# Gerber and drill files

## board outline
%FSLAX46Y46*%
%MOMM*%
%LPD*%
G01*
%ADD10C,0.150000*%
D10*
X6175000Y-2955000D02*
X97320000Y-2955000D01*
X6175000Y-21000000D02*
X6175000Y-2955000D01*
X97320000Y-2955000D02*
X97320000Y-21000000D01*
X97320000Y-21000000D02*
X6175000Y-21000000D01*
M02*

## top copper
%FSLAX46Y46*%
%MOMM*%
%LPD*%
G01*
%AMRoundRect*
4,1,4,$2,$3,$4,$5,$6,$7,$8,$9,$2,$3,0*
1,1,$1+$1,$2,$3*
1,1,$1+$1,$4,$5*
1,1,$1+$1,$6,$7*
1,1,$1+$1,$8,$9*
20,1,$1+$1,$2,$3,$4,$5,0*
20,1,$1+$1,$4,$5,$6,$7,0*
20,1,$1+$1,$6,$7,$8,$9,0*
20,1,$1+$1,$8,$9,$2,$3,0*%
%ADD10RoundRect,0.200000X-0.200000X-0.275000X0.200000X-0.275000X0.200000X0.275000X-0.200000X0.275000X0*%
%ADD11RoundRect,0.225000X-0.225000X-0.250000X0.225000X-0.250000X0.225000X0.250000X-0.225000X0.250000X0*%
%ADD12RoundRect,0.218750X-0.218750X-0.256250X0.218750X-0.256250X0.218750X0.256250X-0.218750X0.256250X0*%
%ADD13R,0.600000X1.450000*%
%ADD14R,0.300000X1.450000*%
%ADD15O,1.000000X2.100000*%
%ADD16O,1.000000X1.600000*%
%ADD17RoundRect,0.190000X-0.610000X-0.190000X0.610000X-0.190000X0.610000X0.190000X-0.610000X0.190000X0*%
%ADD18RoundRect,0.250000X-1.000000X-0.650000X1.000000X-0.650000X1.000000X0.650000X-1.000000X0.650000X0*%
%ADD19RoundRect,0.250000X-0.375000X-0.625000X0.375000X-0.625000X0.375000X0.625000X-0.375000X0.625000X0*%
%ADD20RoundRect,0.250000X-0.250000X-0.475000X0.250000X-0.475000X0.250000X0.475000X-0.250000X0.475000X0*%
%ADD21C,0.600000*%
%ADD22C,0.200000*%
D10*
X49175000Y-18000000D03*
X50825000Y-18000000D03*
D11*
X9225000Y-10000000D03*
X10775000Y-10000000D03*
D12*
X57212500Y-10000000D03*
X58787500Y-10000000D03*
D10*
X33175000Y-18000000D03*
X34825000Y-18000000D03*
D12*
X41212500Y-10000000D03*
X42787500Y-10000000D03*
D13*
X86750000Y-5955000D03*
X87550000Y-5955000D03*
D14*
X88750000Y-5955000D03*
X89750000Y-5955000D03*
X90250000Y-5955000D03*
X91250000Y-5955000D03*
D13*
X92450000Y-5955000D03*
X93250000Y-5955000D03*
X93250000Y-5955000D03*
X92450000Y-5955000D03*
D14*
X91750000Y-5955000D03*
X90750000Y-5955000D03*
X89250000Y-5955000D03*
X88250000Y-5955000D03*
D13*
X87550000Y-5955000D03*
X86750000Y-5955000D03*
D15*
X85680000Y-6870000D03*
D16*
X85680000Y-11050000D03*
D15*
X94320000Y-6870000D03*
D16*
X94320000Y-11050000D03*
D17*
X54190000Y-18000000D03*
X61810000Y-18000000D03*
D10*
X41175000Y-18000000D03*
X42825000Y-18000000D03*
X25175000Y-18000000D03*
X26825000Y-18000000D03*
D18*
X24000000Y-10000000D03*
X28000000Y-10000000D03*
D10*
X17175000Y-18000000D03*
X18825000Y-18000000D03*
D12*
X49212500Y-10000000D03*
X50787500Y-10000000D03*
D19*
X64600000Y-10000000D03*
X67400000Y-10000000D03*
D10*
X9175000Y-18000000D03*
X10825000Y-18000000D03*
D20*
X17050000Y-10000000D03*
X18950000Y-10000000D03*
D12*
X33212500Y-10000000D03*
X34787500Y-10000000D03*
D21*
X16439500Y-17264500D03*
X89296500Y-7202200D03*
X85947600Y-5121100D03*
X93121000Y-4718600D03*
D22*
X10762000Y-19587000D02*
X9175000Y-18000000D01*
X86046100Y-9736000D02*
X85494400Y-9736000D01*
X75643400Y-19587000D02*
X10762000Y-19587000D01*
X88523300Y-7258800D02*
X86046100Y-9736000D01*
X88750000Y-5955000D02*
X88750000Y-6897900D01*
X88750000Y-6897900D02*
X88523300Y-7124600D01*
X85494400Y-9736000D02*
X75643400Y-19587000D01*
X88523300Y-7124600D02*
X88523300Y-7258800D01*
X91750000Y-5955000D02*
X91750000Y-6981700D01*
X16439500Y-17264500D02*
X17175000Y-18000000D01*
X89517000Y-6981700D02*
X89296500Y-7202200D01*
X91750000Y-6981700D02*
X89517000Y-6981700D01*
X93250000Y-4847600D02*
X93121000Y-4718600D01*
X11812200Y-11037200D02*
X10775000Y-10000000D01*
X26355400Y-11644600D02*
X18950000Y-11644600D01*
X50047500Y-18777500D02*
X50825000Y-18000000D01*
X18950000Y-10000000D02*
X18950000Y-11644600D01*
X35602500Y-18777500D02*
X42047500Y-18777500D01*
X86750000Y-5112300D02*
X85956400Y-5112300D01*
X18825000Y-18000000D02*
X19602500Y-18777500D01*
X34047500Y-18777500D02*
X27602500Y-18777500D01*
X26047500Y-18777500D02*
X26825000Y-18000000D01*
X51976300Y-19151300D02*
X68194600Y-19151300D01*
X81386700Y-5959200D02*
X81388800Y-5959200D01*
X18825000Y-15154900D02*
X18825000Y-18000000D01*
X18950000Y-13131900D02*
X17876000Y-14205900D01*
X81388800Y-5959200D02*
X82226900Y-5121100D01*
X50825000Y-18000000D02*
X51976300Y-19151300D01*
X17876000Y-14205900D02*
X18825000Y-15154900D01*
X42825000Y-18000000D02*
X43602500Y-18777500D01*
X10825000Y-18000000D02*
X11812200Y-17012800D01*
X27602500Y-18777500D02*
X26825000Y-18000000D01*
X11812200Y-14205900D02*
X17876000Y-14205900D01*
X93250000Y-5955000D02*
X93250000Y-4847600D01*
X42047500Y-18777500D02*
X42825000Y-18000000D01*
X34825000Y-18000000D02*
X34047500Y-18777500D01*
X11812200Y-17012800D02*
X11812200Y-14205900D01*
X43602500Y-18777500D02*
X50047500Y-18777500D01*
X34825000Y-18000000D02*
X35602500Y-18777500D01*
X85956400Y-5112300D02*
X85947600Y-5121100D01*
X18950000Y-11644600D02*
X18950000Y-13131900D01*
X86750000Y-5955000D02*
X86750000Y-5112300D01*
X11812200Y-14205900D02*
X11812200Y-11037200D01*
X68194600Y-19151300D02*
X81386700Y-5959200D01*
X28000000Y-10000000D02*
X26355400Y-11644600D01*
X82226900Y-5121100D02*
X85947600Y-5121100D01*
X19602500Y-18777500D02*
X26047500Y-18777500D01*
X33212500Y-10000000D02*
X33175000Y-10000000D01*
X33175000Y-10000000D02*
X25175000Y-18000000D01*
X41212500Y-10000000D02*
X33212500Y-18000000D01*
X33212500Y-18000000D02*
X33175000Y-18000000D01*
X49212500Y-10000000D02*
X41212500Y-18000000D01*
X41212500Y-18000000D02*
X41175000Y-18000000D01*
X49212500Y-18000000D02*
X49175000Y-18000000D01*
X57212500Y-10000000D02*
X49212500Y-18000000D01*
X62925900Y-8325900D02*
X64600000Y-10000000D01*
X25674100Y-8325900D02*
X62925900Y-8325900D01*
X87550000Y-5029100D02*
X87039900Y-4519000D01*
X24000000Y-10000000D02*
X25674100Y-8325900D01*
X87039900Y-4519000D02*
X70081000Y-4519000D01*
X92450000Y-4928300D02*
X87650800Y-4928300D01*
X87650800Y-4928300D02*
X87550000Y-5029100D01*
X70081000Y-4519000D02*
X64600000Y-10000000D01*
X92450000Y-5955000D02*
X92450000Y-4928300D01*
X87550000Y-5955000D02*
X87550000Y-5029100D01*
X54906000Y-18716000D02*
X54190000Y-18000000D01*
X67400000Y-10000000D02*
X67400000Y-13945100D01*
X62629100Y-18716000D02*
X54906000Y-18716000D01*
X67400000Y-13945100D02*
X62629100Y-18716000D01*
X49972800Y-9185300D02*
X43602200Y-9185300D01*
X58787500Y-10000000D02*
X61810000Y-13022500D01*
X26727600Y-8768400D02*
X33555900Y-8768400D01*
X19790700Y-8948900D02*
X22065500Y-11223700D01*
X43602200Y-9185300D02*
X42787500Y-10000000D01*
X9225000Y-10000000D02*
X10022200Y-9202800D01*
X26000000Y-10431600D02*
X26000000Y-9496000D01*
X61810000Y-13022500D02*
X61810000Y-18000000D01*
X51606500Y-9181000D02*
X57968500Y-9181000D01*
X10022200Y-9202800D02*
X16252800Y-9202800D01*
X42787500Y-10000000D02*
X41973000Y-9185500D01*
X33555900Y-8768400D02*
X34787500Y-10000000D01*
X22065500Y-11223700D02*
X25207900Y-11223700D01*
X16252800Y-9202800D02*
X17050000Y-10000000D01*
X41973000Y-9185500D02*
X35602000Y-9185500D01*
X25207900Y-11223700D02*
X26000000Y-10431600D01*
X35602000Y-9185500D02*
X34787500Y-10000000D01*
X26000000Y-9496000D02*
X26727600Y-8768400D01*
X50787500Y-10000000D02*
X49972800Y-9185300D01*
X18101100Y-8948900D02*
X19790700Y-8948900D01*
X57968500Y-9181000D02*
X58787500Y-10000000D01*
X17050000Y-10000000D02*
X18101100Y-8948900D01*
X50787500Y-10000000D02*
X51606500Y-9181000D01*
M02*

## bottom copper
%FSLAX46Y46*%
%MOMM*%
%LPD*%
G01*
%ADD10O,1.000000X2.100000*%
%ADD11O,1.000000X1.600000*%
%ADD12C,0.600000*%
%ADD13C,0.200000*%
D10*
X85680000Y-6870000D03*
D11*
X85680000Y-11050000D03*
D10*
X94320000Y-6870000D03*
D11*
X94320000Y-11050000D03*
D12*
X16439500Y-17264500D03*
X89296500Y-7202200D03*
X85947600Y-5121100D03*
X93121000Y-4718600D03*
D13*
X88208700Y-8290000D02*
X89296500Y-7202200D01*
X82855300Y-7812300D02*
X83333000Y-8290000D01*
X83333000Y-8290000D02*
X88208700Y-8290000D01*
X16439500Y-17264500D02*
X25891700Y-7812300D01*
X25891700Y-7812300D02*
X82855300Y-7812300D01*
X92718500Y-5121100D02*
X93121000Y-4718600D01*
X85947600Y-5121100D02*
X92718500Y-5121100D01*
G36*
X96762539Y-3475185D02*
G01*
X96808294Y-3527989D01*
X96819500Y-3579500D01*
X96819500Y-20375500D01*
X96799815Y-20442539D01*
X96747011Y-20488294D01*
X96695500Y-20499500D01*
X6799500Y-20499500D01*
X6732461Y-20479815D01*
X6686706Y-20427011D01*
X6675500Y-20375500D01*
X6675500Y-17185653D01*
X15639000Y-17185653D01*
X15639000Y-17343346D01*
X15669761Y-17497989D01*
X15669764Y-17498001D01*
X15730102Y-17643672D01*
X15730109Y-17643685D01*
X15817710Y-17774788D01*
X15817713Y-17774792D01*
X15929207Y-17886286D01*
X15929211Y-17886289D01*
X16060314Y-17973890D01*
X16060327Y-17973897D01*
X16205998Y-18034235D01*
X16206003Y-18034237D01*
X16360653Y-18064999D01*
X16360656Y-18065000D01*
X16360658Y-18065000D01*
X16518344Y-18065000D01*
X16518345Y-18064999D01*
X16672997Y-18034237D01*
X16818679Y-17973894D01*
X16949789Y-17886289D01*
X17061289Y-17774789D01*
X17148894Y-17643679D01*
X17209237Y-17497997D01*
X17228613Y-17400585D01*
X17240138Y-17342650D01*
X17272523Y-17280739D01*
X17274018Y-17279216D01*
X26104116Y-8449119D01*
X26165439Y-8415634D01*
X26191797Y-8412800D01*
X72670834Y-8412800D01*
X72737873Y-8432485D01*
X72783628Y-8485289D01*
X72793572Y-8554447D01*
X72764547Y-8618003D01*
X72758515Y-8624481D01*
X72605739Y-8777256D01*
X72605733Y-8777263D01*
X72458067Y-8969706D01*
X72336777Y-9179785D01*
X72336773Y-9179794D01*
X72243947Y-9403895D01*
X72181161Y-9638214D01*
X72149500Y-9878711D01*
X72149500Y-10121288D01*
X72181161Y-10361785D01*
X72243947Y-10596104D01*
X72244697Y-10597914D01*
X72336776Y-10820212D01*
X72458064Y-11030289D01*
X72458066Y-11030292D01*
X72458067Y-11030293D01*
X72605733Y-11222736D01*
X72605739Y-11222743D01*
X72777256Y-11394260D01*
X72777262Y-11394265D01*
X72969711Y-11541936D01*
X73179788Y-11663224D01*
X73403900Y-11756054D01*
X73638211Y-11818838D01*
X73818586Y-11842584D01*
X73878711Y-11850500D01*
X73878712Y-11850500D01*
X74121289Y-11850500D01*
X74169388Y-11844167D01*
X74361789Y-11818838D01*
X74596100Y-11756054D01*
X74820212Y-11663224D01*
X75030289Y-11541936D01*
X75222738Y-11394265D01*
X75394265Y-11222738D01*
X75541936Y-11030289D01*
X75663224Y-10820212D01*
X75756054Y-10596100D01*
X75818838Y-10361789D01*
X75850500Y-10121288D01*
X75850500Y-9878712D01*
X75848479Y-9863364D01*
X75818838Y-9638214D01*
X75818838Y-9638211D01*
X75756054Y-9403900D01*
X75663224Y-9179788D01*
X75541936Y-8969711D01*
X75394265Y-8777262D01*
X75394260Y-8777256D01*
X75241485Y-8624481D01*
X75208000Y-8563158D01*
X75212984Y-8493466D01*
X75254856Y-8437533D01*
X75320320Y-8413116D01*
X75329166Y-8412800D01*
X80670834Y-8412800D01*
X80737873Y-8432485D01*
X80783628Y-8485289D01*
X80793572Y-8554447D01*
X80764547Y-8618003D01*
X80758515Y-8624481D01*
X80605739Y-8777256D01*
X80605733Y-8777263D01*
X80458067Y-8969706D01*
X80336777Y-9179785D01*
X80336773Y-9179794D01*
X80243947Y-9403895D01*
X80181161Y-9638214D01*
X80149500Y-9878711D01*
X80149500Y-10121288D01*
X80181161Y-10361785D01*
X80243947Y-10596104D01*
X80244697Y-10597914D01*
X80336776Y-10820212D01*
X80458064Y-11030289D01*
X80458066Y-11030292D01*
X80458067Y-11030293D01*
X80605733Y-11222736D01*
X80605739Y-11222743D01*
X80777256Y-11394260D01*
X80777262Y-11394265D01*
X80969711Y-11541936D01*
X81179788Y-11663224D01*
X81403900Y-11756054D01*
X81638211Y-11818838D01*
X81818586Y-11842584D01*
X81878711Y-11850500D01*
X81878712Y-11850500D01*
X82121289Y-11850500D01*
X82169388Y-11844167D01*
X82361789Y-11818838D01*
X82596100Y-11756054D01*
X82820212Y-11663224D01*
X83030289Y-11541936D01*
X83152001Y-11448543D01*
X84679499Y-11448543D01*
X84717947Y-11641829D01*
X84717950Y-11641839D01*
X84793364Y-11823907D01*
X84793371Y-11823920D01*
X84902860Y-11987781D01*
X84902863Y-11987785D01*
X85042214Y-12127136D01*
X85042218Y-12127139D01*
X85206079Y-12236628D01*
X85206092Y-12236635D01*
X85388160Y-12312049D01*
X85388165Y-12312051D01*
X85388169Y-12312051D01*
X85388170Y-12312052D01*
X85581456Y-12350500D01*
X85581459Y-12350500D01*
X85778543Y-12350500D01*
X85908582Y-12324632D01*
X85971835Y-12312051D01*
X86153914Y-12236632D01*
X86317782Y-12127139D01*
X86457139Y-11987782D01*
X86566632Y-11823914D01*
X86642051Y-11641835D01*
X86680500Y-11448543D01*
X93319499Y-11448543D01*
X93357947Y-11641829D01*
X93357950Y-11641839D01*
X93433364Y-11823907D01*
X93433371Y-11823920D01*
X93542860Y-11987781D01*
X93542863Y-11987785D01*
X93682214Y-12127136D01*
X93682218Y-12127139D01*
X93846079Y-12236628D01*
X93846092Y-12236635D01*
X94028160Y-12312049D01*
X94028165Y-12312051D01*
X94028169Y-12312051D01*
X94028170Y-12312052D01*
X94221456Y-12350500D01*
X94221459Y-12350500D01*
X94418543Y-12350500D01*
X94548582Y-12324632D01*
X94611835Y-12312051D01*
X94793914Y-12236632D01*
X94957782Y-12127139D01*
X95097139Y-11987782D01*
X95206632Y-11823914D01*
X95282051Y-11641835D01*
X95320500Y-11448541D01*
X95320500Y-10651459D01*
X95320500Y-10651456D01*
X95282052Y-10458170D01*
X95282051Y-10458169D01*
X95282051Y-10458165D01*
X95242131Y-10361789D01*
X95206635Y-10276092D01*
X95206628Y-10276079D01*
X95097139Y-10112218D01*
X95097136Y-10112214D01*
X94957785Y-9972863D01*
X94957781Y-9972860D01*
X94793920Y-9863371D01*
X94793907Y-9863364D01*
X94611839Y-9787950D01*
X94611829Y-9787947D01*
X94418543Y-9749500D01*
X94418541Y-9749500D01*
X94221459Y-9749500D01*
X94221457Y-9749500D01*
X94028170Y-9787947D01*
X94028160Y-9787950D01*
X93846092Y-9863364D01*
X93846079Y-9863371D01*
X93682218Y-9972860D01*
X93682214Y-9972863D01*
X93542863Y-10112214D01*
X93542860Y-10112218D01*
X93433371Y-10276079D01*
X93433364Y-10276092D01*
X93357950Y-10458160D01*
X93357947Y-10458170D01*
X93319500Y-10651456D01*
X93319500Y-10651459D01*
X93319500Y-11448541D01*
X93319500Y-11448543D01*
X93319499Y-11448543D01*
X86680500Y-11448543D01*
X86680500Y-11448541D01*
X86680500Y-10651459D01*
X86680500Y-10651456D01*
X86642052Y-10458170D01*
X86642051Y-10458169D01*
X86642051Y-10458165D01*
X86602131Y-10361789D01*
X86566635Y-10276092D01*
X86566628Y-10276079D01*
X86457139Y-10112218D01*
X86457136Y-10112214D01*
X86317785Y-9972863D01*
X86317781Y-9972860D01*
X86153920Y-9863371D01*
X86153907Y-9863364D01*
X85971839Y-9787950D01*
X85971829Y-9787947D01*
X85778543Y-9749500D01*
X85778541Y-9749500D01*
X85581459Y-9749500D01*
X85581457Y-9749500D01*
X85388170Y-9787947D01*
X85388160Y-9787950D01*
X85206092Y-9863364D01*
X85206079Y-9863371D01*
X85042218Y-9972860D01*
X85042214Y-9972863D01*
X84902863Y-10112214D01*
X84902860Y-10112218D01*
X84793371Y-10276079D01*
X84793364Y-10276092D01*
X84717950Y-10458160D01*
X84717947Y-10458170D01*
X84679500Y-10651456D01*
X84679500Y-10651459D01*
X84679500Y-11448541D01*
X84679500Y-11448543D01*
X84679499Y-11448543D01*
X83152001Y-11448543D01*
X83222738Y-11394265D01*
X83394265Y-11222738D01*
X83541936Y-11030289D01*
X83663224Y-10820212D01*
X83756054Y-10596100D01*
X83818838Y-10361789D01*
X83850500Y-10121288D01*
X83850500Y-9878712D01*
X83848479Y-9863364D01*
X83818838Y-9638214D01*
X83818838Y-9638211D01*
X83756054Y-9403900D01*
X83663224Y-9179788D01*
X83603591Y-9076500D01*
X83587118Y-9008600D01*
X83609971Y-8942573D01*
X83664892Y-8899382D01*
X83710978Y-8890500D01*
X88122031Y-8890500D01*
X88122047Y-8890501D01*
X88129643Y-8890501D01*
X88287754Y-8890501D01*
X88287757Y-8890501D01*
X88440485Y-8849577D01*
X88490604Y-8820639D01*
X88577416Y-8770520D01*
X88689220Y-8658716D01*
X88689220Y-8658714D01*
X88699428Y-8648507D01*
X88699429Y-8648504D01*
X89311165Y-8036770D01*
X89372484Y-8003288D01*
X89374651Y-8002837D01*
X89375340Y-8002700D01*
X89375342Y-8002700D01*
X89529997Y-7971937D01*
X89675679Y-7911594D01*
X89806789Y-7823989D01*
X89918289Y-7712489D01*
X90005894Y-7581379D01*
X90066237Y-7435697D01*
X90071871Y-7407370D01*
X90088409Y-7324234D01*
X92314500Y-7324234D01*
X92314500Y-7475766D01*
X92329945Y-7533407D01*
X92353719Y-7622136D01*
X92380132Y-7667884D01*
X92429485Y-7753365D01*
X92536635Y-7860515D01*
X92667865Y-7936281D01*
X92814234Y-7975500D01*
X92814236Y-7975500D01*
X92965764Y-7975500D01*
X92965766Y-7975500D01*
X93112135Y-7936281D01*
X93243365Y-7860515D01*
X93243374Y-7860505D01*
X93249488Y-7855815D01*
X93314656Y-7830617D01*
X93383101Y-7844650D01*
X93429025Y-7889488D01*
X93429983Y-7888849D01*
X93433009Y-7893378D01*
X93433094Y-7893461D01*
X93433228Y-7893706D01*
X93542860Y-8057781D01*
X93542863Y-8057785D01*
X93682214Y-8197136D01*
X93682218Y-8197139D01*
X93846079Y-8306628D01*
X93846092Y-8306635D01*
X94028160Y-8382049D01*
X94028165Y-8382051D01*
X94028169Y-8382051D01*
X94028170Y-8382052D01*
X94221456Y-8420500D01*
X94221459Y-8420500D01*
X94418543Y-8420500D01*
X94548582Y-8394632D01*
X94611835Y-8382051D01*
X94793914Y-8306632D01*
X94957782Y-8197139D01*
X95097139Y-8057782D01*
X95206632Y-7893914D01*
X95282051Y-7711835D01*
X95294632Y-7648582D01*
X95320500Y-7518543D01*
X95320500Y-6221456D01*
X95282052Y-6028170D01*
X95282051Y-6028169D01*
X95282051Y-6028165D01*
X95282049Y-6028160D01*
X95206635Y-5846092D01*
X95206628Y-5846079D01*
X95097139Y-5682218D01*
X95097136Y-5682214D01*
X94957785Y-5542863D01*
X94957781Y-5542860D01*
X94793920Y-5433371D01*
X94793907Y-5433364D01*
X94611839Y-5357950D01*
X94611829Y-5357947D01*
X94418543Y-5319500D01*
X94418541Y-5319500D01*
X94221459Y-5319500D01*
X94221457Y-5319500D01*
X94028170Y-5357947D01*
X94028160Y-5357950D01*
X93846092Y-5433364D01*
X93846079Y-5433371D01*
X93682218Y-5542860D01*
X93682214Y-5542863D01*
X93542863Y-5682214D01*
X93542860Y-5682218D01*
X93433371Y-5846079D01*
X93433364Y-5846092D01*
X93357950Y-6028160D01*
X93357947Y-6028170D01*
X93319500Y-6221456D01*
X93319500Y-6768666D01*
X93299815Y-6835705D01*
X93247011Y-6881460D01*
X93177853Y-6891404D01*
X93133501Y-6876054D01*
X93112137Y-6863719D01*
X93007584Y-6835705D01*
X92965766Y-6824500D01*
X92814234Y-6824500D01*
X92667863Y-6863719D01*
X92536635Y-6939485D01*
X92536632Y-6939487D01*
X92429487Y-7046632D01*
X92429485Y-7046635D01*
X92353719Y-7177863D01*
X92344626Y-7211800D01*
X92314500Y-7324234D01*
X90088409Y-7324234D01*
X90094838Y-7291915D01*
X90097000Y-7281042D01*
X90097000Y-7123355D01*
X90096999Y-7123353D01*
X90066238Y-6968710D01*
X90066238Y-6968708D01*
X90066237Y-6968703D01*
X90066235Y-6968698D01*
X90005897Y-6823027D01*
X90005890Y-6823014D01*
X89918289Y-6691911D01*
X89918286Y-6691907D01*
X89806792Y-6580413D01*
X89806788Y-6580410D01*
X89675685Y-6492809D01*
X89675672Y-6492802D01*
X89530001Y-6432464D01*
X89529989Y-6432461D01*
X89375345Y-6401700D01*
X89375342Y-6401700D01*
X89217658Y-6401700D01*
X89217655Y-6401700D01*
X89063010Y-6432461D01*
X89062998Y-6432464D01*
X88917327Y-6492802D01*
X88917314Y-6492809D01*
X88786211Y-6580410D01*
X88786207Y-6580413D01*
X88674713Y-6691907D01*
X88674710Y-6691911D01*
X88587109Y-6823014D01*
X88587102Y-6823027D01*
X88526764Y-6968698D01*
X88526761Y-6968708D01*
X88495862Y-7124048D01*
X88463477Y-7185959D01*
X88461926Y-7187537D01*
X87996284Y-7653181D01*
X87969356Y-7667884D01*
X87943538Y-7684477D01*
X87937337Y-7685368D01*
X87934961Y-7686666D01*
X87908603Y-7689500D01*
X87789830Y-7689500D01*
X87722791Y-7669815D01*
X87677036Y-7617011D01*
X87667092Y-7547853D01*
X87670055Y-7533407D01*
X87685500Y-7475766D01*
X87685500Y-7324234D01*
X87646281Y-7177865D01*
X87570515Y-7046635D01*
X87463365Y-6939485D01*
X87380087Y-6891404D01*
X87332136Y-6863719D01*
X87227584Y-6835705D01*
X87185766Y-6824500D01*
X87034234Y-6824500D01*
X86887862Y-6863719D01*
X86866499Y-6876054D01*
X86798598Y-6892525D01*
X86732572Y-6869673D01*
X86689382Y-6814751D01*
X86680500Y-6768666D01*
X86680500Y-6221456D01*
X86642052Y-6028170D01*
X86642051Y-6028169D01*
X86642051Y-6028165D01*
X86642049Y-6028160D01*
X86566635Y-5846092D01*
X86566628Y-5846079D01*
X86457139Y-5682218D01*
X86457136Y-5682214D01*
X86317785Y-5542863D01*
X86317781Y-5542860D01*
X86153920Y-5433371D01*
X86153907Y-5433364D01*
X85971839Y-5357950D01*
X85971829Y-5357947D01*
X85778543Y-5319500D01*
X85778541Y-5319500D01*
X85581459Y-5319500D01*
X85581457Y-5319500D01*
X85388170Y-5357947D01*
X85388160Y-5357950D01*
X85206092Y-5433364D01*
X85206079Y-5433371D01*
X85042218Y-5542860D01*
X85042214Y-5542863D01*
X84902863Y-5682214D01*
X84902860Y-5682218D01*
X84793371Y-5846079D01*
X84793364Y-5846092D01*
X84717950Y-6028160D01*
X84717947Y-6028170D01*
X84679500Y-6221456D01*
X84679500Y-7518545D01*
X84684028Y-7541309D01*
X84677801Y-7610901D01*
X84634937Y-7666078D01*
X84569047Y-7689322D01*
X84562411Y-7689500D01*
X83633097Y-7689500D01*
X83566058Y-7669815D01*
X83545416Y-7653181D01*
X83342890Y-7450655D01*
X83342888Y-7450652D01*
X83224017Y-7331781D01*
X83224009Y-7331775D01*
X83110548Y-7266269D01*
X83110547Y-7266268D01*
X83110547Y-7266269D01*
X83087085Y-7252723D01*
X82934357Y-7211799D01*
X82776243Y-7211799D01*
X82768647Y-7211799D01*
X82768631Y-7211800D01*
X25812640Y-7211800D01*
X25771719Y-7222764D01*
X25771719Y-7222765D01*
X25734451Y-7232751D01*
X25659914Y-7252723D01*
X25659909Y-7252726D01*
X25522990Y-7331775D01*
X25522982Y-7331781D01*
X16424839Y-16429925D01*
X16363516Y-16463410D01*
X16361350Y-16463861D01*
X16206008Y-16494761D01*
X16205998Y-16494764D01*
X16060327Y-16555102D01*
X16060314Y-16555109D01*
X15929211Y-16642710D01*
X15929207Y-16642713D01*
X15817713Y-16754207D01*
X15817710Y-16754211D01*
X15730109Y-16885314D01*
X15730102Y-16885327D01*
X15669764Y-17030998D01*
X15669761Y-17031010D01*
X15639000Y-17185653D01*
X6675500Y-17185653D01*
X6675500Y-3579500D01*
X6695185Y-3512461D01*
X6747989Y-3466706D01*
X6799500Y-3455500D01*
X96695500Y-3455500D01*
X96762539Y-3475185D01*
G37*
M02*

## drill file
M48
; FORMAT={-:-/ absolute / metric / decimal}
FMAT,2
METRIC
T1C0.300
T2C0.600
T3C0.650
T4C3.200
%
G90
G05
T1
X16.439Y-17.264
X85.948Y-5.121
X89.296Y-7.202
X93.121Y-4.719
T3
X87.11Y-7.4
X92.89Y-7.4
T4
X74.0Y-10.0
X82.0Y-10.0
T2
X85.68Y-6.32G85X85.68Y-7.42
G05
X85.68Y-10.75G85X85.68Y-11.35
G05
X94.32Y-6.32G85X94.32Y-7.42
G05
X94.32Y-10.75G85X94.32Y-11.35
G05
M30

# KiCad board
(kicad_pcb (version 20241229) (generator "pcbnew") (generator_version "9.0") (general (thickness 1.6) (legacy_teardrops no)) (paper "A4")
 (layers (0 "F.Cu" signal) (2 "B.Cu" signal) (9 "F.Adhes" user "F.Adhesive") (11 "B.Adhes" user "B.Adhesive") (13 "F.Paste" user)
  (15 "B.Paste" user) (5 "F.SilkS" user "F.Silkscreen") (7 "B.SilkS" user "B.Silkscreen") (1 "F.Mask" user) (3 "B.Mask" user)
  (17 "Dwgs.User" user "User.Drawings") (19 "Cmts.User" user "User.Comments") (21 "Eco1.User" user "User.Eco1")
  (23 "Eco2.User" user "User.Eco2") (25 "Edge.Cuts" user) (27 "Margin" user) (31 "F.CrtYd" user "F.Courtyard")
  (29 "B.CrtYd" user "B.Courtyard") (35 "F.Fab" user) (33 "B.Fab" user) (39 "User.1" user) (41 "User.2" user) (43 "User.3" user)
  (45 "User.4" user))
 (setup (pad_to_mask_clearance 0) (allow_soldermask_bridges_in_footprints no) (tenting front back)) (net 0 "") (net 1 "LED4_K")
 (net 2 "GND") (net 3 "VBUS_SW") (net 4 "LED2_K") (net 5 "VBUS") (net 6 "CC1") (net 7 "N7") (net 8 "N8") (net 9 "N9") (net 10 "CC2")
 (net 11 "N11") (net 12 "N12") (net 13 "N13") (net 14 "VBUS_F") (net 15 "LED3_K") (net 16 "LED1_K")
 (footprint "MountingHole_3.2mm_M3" (layer "F.Cu") (at 74 10)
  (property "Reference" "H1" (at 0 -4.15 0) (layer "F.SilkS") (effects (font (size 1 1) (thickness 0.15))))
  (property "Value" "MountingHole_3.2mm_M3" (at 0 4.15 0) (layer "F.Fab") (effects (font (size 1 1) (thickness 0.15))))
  (pad "" np_thru_hole circle (at 0 0) (size 3.2 3.2) (drill 3.2) (layers "*.Cu" "*.Mask")))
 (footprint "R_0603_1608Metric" (layer "F.Cu") (at 50 18)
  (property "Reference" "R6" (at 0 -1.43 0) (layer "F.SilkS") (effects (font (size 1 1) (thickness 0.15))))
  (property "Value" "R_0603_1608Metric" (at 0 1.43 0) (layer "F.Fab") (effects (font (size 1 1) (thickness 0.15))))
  (pad "1" smd roundrect (at -0.825 0) (size 0.8 0.95) (layers "F.Cu" "F.Mask" "F.Paste") (roundrect_rratio 0.25) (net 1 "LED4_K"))
  (pad "2" smd roundrect (at 0.825 0) (size 0.8 0.95) (layers "F.Cu" "F.Mask" "F.Paste") (roundrect_rratio 0.25) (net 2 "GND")))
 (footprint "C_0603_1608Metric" (layer "F.Cu") (at 10 10)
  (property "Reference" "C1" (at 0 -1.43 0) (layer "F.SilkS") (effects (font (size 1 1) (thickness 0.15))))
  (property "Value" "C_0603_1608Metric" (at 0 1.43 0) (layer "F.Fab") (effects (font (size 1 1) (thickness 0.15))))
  (pad "1" smd roundrect (at -0.775 0) (size 0.9 0.95) (layers "F.Cu" "F.Mask" "F.Paste") (roundrect_rratio 0.25) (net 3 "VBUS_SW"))
  (pad "2" smd roundrect (at 0.775 0) (size 0.9 0.95) (layers "F.Cu" "F.Mask" "F.Paste") (roundrect_rratio 0.25) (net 2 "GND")))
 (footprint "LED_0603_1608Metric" (layer "F.Cu") (at 58 10)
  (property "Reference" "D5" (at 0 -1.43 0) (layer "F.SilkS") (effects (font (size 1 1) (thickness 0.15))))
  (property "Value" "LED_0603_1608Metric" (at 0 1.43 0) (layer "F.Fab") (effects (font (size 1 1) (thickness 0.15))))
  (pad "1" smd roundrect (at -0.7875 0) (size 0.875 0.95) (layers "F.Cu" "F.Mask" "F.Paste") (roundrect_rratio 0.25) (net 1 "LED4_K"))
  (pad "2" smd roundrect (at 0.7875 0) (size 0.875 0.95) (layers "F.Cu" "F.Mask" "F.Paste") (roundrect_rratio 0.25) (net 3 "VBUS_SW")))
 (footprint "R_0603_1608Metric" (layer "F.Cu") (at 34 18)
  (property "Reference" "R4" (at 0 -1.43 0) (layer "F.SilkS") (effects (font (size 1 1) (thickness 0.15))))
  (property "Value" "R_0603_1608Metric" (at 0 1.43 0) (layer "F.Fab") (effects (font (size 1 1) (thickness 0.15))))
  (pad "1" smd roundrect (at -0.825 0) (size 0.8 0.95) (layers "F.Cu" "F.Mask" "F.Paste") (roundrect_rratio 0.25) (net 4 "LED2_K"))
  (pad "2" smd roundrect (at 0.825 0) (size 0.8 0.95) (layers "F.Cu" "F.Mask" "F.Paste") (roundrect_rratio 0.25) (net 2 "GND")))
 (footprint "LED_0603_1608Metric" (layer "F.Cu") (at 42 10)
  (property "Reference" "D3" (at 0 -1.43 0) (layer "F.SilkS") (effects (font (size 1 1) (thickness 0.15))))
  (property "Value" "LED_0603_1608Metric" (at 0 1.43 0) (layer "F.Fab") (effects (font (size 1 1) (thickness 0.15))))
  (pad "1" smd roundrect (at -0.7875 0) (size 0.875 0.95) (layers "F.Cu" "F.Mask" "F.Paste") (roundrect_rratio 0.25) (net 4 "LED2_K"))
  (pad "2" smd roundrect (at 0.7875 0) (size 0.875 0.95) (layers "F.Cu" "F.Mask" "F.Paste") (roundrect_rratio 0.25) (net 3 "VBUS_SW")))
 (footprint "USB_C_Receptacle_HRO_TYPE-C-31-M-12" (layer "F.Cu") (at 90 10)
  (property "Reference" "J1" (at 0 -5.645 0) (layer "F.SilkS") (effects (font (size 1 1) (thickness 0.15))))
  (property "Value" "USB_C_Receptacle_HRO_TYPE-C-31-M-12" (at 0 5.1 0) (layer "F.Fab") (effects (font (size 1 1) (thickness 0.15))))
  (pad "" np_thru_hole circle (at -2.89 -2.6) (size 0.65 0.65) (drill 0.65) (layers "*.Cu" "*.Mask"))
  (pad "" np_thru_hole circle (at 2.89 -2.6) (size 0.65 0.65) (drill 0.65) (layers "*.Cu" "*.Mask"))
  (pad "A1" smd rect (at -3.25 -4.045) (size 0.6 1.45) (layers "F.Cu" "F.Mask" "F.Paste") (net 2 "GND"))
  (pad "A4" smd rect (at -2.45 -4.045) (size 0.6 1.45) (layers "F.Cu" "F.Mask" "F.Paste") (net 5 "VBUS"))
  (pad "A5" smd rect (at -1.25 -4.045) (size 0.3 1.45) (layers "F.Cu" "F.Mask" "F.Paste") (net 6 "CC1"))
  (pad "A6" smd rect (at -0.25 -4.045) (size 0.3 1.45) (layers "F.Cu" "F.Mask" "F.Paste") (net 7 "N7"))
  (pad "A7" smd rect (at 0.25 -4.045) (size 0.3 1.45) (layers "F.Cu" "F.Mask" "F.Paste") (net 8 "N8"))
  (pad "A8" smd rect (at 1.25 -4.045) (size 0.3 1.45) (layers "F.Cu" "F.Mask" "F.Paste") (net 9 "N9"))
  (pad "A9" smd rect (at 2.45 -4.045) (size 0.6 1.45) (layers "F.Cu" "F.Mask" "F.Paste") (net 5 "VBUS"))
  (pad "A12" smd rect (at 3.25 -4.045) (size 0.6 1.45) (layers "F.Cu" "F.Mask" "F.Paste") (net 2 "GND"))
  (pad "B1" smd rect (at 3.25 -4.045) (size 0.6 1.45) (layers "F.Cu" "F.Mask" "F.Paste") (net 2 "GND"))
  (pad "B4" smd rect (at 2.45 -4.045) (size 0.6 1.45) (layers "F.Cu" "F.Mask" "F.Paste") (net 5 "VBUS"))
  (pad "B5" smd rect (at 1.75 -4.045) (size 0.3 1.45) (layers "F.Cu" "F.Mask" "F.Paste") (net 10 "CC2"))
  (pad "B6" smd rect (at 0.75 -4.045) (size 0.3 1.45) (layers "F.Cu" "F.Mask" "F.Paste") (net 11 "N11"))
  (pad "B7" smd rect (at -0.75 -4.045) (size 0.3 1.45) (layers "F.Cu" "F.Mask" "F.Paste") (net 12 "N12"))
  (pad "B8" smd rect (at -1.75 -4.045) (size 0.3 1.45) (layers "F.Cu" "F.Mask" "F.Paste") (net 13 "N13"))
  (pad "B9" smd rect (at -2.45 -4.045) (size 0.6 1.45) (layers "F.Cu" "F.Mask" "F.Paste") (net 5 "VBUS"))
  (pad "B12" smd rect (at -3.25 -4.045) (size 0.6 1.45) (layers "F.Cu" "F.Mask" "F.Paste") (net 2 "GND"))
  (pad "S1" thru_hole oval (at -4.32 -3.13) (size 1 2.1) (drill oval 0.6 1.7) (layers "*.Cu" "*.Mask") (remove_unused_layers no))
  (pad "S1" thru_hole oval (at -4.32 1.05) (size 1 1.6) (drill oval 0.6 1.2) (layers "*.Cu" "*.Mask") (remove_unused_layers no))
  (pad "S1" thru_hole oval (at 4.32 -3.13) (size 1 2.1) (drill oval 0.6 1.7) (layers "*.Cu" "*.Mask") (remove_unused_layers no))
  (pad "S1" thru_hole oval (at 4.32 1.05) (size 1 1.6) (drill oval 0.6 1.2) (layers "*.Cu" "*.Mask") (remove_unused_layers no)))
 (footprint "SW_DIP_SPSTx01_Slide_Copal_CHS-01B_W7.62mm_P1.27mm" (layer "F.Cu") (at 58 18)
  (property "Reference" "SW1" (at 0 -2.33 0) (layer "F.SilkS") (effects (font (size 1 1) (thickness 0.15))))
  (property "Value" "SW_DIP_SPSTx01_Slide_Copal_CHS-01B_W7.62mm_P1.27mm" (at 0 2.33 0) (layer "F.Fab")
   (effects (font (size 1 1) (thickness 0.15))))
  (pad "1" smd roundrect (at -3.81 0) (size 1.6 0.76) (layers "F.Cu" "F.Mask" "F.Paste") (roundrect_rratio 0.25) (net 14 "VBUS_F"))
  (pad "2" smd roundrect (at 3.81 0) (size 1.6 0.76) (layers "F.Cu" "F.Mask" "F.Paste") (roundrect_rratio 0.25) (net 3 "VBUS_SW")))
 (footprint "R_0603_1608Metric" (layer "F.Cu") (at 42 18)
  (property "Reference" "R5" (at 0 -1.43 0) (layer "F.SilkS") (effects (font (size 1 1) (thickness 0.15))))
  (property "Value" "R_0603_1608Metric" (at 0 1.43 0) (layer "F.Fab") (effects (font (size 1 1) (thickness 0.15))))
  (pad "1" smd roundrect (at -0.825 0) (size 0.8 0.95) (layers "F.Cu" "F.Mask" "F.Paste") (roundrect_rratio 0.25) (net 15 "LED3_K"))
  (pad "2" smd roundrect (at 0.825 0) (size 0.8 0.95) (layers "F.Cu" "F.Mask" "F.Paste") (roundrect_rratio 0.25) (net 2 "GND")))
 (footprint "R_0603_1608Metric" (layer "F.Cu") (at 26 18)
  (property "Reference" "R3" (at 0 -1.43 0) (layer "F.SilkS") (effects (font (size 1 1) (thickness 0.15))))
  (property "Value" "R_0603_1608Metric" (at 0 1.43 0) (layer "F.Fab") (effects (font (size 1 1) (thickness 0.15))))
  (pad "1" smd roundrect (at -0.825 0) (size 0.8 0.95) (layers "F.Cu" "F.Mask" "F.Paste") (roundrect_rratio 0.25) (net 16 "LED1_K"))
  (pad "2" smd roundrect (at 0.825 0) (size 0.8 0.95) (layers "F.Cu" "F.Mask" "F.Paste") (roundrect_rratio 0.25) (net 2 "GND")))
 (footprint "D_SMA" (layer "F.Cu") (at 26 10)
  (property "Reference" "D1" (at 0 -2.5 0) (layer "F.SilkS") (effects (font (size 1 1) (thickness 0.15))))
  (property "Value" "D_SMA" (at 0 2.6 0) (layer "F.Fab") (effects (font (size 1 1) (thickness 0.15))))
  (pad "1" smd roundrect (at -2 0) (size 2.5 1.8) (layers "F.Cu" "F.Mask" "F.Paste") (roundrect_rratio 0.1388888889) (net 5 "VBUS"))
  (pad "2" smd roundrect (at 2 0) (size 2.5 1.8) (layers "F.Cu" "F.Mask" "F.Paste") (roundrect_rratio 0.1388888889) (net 2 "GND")))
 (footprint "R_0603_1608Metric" (layer "F.Cu") (at 18 18)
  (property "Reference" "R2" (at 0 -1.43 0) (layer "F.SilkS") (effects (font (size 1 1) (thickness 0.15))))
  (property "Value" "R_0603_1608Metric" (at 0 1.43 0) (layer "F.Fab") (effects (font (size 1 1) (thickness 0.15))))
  (pad "1" smd roundrect (at -0.825 0) (size 0.8 0.95) (layers "F.Cu" "F.Mask" "F.Paste") (roundrect_rratio 0.25) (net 10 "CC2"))
  (pad "2" smd roundrect (at 0.825 0) (size 0.8 0.95) (layers "F.Cu" "F.Mask" "F.Paste") (roundrect_rratio 0.25) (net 2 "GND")))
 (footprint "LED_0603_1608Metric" (layer "F.Cu") (at 50 10)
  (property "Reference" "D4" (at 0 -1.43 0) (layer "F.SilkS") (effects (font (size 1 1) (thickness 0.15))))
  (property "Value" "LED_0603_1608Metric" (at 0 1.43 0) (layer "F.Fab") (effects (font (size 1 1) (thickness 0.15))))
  (pad "1" smd roundrect (at -0.7875 0) (size 0.875 0.95) (layers "F.Cu" "F.Mask" "F.Paste") (roundrect_rratio 0.25) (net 15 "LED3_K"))
  (pad "2" smd roundrect (at 0.7875 0) (size 0.875 0.95) (layers "F.Cu" "F.Mask" "F.Paste") (roundrect_rratio 0.25) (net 3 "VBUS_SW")))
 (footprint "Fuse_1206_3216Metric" (layer "F.Cu") (at 66 10)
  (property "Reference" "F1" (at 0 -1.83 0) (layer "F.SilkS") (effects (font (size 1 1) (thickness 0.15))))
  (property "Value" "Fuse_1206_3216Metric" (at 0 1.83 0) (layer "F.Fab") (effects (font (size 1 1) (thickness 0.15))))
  (pad "1" smd roundrect (at -1.4 0) (size 1.25 1.75) (layers "F.Cu" "F.Mask" "F.Paste") (roundrect_rratio 0.2) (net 5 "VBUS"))
  (pad "2" smd roundrect (at 1.4 0) (size 1.25 1.75) (layers "F.Cu" "F.Mask" "F.Paste") (roundrect_rratio 0.2) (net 14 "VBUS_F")))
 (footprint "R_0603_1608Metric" (layer "F.Cu") (at 10 18)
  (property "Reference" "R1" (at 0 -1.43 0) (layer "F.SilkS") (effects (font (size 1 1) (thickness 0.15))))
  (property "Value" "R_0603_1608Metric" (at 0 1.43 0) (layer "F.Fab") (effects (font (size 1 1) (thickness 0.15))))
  (pad "1" smd roundrect (at -0.825 0) (size 0.8 0.95) (layers "F.Cu" "F.Mask" "F.Paste") (roundrect_rratio 0.25) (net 6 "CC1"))
  (pad "2" smd roundrect (at 0.825 0) (size 0.8 0.95) (layers "F.Cu" "F.Mask" "F.Paste") (roundrect_rratio 0.25) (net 2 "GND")))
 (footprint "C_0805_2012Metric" (layer "F.Cu") (at 18 10)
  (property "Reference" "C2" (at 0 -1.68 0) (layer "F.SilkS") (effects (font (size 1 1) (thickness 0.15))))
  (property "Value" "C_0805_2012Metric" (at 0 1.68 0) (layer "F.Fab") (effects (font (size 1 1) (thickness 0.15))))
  (pad "1" smd roundrect (at -0.95 0) (size 1 1.45) (layers "F.Cu" "F.Mask" "F.Paste") (roundrect_rratio 0.25) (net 3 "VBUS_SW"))
  (pad "2" smd roundrect (at 0.95 0) (size 1 1.45) (layers "F.Cu" "F.Mask" "F.Paste") (roundrect_rratio 0.25) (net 2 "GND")))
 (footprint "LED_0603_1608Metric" (layer "F.Cu") (at 34 10)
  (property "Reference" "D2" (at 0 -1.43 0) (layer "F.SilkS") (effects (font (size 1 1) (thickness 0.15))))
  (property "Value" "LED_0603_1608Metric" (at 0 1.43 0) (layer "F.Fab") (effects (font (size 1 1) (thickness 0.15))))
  (pad "1" smd roundrect (at -0.7875 0) (size 0.875 0.95) (layers "F.Cu" "F.Mask" "F.Paste") (roundrect_rratio 0.25) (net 16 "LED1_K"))
  (pad "2" smd roundrect (at 0.7875 0) (size 0.875 0.95) (layers "F.Cu" "F.Mask" "F.Paste") (roundrect_rratio 0.25) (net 3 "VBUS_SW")))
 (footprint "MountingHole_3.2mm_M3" (layer "F.Cu") (at 82 10)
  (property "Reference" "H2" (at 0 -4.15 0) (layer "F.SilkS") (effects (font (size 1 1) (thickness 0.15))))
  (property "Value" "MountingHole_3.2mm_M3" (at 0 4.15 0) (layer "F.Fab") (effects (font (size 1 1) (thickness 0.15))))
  (pad "" np_thru_hole circle (at 0 0) (size 3.2 3.2) (drill 3.2) (layers "*.Cu" "*.Mask")))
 (gr_line (start 6.175 2.955) (end 97.32 2.955) (stroke (width 0.15) (type default)) (layer "Edge.Cuts"))
 (gr_line (start 6.175 21) (end 6.175 2.955) (stroke (width 0.15) (type default)) (layer "Edge.Cuts"))
 (gr_line (start 97.32 2.955) (end 97.32 21) (stroke (width 0.15) (type default)) (layer "Edge.Cuts"))
 (gr_line (start 97.32 21) (end 6.175 21) (stroke (width 0.15) (type default)) (layer "Edge.Cuts"))
 (segment (start 10.762 19.587) (end 9.175 18) (width 0.2) (layer "F.Cu") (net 6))
 (segment (start 86.0461 9.736) (end 85.4944 9.736) (width 0.2) (layer "F.Cu") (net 6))
 (segment (start 75.6434 19.587) (end 10.762 19.587) (width 0.2) (layer "F.Cu") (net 6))
 (segment (start 88.5233 7.2588) (end 86.0461 9.736) (width 0.2) (layer "F.Cu") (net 6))
 (segment (start 88.75 5.955) (end 88.75 6.8979) (width 0.2) (layer "F.Cu") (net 6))
 (segment (start 88.75 6.8979) (end 88.5233 7.1246) (width 0.2) (layer "F.Cu") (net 6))
 (segment (start 85.4944 9.736) (end 75.6434 19.587) (width 0.2) (layer "F.Cu") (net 6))
 (segment (start 88.5233 7.1246) (end 88.5233 7.2588) (width 0.2) (layer "F.Cu") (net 6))
 (segment (start 91.75 5.955) (end 91.75 6.9817) (width 0.2) (layer "F.Cu") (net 10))
 (segment (start 16.4395 17.2645) (end 17.175 18) (width 0.2) (layer "F.Cu") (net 10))
 (segment (start 89.517 6.9817) (end 89.2965 7.2022) (width 0.2) (layer "F.Cu") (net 10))
 (segment (start 91.75 6.9817) (end 89.517 6.9817) (width 0.2) (layer "F.Cu") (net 10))
 (via (at 16.4395 17.2645) (size 0.6) (drill 0.3) (layers "F.Cu" "B.Cu") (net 10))
 (via (at 89.2965 7.2022) (size 0.6) (drill 0.3) (layers "F.Cu" "B.Cu") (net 10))
 (segment (start 88.2087 8.29) (end 89.2965 7.2022) (width 0.2) (layer "B.Cu") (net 10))
 (segment (start 82.8553 7.8123) (end 83.333 8.29) (width 0.2) (layer "B.Cu") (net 10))
 (segment (start 83.333 8.29) (end 88.2087 8.29) (width 0.2) (layer "B.Cu") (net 10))
 (segment (start 16.4395 17.2645) (end 25.8917 7.8123) (width 0.2) (layer "B.Cu") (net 10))
 (segment (start 25.8917 7.8123) (end 82.8553 7.8123) (width 0.2) (layer "B.Cu") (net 10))
 (segment (start 93.25 4.8476) (end 93.121 4.7186) (width 0.2) (layer "F.Cu") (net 2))
 (segment (start 11.8122 11.0372) (end 10.775 10) (width 0.2) (layer "F.Cu") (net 2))
 (segment (start 26.3554 11.6446) (end 18.95 11.6446) (width 0.2) (layer "F.Cu") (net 2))
 (segment (start 50.0475 18.7775) (end 50.825 18) (width 0.2) (layer "F.Cu") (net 2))
 (segment (start 18.95 10) (end 18.95 11.6446) (width 0.2) (layer "F.Cu") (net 2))
 (segment (start 35.6025 18.7775) (end 42.0475 18.7775) (width 0.2) (layer "F.Cu") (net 2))
 (segment (start 86.75 5.1123) (end 85.9564 5.1123) (width 0.2) (layer "F.Cu") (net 2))
 (segment (start 18.825 18) (end 19.6025 18.7775) (width 0.2) (layer "F.Cu") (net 2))
 (segment (start 34.0475 18.7775) (end 27.6025 18.7775) (width 0.2) (layer "F.Cu") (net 2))
 (segment (start 26.0475 18.7775) (end 26.825 18) (width 0.2) (layer "F.Cu") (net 2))
 (segment (start 51.9763 19.1513) (end 68.1946 19.1513) (width 0.2) (layer "F.Cu") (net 2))
 (segment (start 81.3867 5.9592) (end 81.3888 5.9592) (width 0.2) (layer "F.Cu") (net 2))
 (segment (start 18.825 15.1549) (end 18.825 18) (width 0.2) (layer "F.Cu") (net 2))
 (segment (start 18.95 13.1319) (end 17.876 14.2059) (width 0.2) (layer "F.Cu") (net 2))
 (segment (start 81.3888 5.9592) (end 82.2269 5.1211) (width 0.2) (layer "F.Cu") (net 2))
 (segment (start 50.825 18) (end 51.9763 19.1513) (width 0.2) (layer "F.Cu") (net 2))
 (segment (start 17.876 14.2059) (end 18.825 15.1549) (width 0.2) (layer "F.Cu") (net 2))
 (segment (start 42.825 18) (end 43.6025 18.7775) (width 0.2) (layer "F.Cu") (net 2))
 (segment (start 10.825 18) (end 11.8122 17.0128) (width 0.2) (layer "F.Cu") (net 2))
 (segment (start 27.6025 18.7775) (end 26.825 18) (width 0.2) (layer "F.Cu") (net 2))
 (segment (start 11.8122 14.2059) (end 17.876 14.2059) (width 0.2) (layer "F.Cu") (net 2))
 (segment (start 93.25 5.955) (end 93.25 4.8476) (width 0.2) (layer "F.Cu") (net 2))
 (segment (start 42.0475 18.7775) (end 42.825 18) (width 0.2) (layer "F.Cu") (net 2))
 (segment (start 34.825 18) (end 34.0475 18.7775) (width 0.2) (layer "F.Cu") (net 2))
 (segment (start 11.8122 17.0128) (end 11.8122 14.2059) (width 0.2) (layer "F.Cu") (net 2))
 (segment (start 43.6025 18.7775) (end 50.0475 18.7775) (width 0.2) (layer "F.Cu") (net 2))
 (segment (start 34.825 18) (end 35.6025 18.7775) (width 0.2) (layer "F.Cu") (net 2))
 (segment (start 85.9564 5.1123) (end 85.9476 5.1211) (width 0.2) (layer "F.Cu") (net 2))
 (segment (start 18.95 11.6446) (end 18.95 13.1319) (width 0.2) (layer "F.Cu") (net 2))
 (segment (start 86.75 5.955) (end 86.75 5.1123) (width 0.2) (layer "F.Cu") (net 2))
 (segment (start 11.8122 14.2059) (end 11.8122 11.0372) (width 0.2) (layer "F.Cu") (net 2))
 (segment (start 68.1946 19.1513) (end 81.3867 5.9592) (width 0.2) (layer "F.Cu") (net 2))
 (segment (start 28 10) (end 26.3554 11.6446) (width 0.2) (layer "F.Cu") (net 2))
 (segment (start 82.2269 5.1211) (end 85.9476 5.1211) (width 0.2) (layer "F.Cu") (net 2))
 (segment (start 19.6025 18.7775) (end 26.0475 18.7775) (width 0.2) (layer "F.Cu") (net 2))
 (via (at 85.9476 5.1211) (size 0.6) (drill 0.3) (layers "F.Cu" "B.Cu") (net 2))
 (via (at 93.121 4.7186) (size 0.6) (drill 0.3) (layers "F.Cu" "B.Cu") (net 2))
 (segment (start 92.7185 5.1211) (end 93.121 4.7186) (width 0.2) (layer "B.Cu") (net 2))
 (segment (start 85.9476 5.1211) (end 92.7185 5.1211) (width 0.2) (layer "B.Cu") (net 2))
 (segment (start 33.2125 10) (end 33.175 10) (width 0.2) (layer "F.Cu") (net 16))
 (segment (start 33.175 10) (end 25.175 18) (width 0.2) (layer "F.Cu") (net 16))
 (segment (start 41.2125 10) (end 33.2125 18) (width 0.2) (layer "F.Cu") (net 4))
 (segment (start 33.2125 18) (end 33.175 18) (width 0.2) (layer "F.Cu") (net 4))
 (segment (start 49.2125 10) (end 41.2125 18) (width 0.2) (layer "F.Cu") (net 15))
 (segment (start 41.2125 18) (end 41.175 18) (width 0.2) (layer "F.Cu") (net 15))
 (segment (start 49.2125 18) (end 49.175 18) (width 0.2) (layer "F.Cu") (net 1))
 (segment (start 57.2125 10) (end 49.2125 18) (width 0.2) (layer "F.Cu") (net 1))
 (segment (start 62.9259 8.3259) (end 64.6 10) (width 0.2) (layer "F.Cu") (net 5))
 (segment (start 25.6741 8.3259) (end 62.9259 8.3259) (width 0.2) (layer "F.Cu") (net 5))
 (segment (start 87.55 5.0291) (end 87.0399 4.519) (width 0.2) (layer "F.Cu") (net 5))
 (segment (start 24 10) (end 25.6741 8.3259) (width 0.2) (layer "F.Cu") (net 5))
 (segment (start 87.0399 4.519) (end 70.081 4.519) (width 0.2) (layer "F.Cu") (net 5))
 (segment (start 92.45 4.9283) (end 87.6508 4.9283) (width 0.2) (layer "F.Cu") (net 5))
 (segment (start 87.6508 4.9283) (end 87.55 5.0291) (width 0.2) (layer "F.Cu") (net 5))
 (segment (start 70.081 4.519) (end 64.6 10) (width 0.2) (layer "F.Cu") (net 5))
 (segment (start 92.45 5.955) (end 92.45 4.9283) (width 0.2) (layer "F.Cu") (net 5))
 (segment (start 87.55 5.955) (end 87.55 5.0291) (width 0.2) (layer "F.Cu") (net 5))
 (segment (start 54.906 18.716) (end 54.19 18) (width 0.2) (layer "F.Cu") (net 14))
 (segment (start 67.4 10) (end 67.4 13.9451) (width 0.2) (layer "F.Cu") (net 14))
 (segment (start 62.6291 18.716) (end 54.906 18.716) (width 0.2) (layer "F.Cu") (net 14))
 (segment (start 67.4 13.9451) (end 62.6291 18.716) (width 0.2) (layer "F.Cu") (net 14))
 (segment (start 49.9728 9.1853) (end 43.6022 9.1853) (width 0.2) (layer "F.Cu") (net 3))
 (segment (start 58.7875 10) (end 61.81 13.0225) (width 0.2) (layer "F.Cu") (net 3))
 (segment (start 26.7276 8.7684) (end 33.5559 8.7684) (width 0.2) (layer "F.Cu") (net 3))
 (segment (start 19.7907 8.9489) (end 22.0655 11.2237) (width 0.2) (layer "F.Cu") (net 3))
 (segment (start 43.6022 9.1853) (end 42.7875 10) (width 0.2) (layer "F.Cu") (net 3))
 (segment (start 9.225 10) (end 10.0222 9.2028) (width 0.2) (layer "F.Cu") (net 3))
 (segment (start 26 10.4316) (end 26 9.496) (width 0.2) (layer "F.Cu") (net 3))
 (segment (start 61.81 13.0225) (end 61.81 18) (width 0.2) (layer "F.Cu") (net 3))
 (segment (start 51.6065 9.181) (end 57.9685 9.181) (width 0.2) (layer "F.Cu") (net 3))
 (segment (start 10.0222 9.2028) (end 16.2528 9.2028) (width 0.2) (layer "F.Cu") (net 3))
 (segment (start 42.7875 10) (end 41.973 9.1855) (width 0.2) (layer "F.Cu") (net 3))
 (segment (start 33.5559 8.7684) (end 34.7875 10) (width 0.2) (layer "F.Cu") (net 3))
 (segment (start 22.0655 11.2237) (end 25.2079 11.2237) (width 0.2) (layer "F.Cu") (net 3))
 (segment (start 16.2528 9.2028) (end 17.05 10) (width 0.2) (layer "F.Cu") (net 3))
 (segment (start 41.973 9.1855) (end 35.602 9.1855) (width 0.2) (layer "F.Cu") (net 3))
 (segment (start 25.2079 11.2237) (end 26 10.4316) (width 0.2) (layer "F.Cu") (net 3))
 (segment (start 35.602 9.1855) (end 34.7875 10) (width 0.2) (layer "F.Cu") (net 3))
 (segment (start 26 9.496) (end 26.7276 8.7684) (width 0.2) (layer "F.Cu") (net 3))
 (segment (start 50.7875 10) (end 49.9728 9.1853) (width 0.2) (layer "F.Cu") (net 3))
 (segment (start 18.1011 8.9489) (end 19.7907 8.9489) (width 0.2) (layer "F.Cu") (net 3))
 (segment (start 57.9685 9.181) (end 58.7875 10) (width 0.2) (layer "F.Cu") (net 3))
 (segment (start 17.05 10) (end 18.1011 8.9489) (width 0.2) (layer "F.Cu") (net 3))
 (segment (start 50.7875 10) (end 51.6065 9.181) (width 0.2) (layer "F.Cu") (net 3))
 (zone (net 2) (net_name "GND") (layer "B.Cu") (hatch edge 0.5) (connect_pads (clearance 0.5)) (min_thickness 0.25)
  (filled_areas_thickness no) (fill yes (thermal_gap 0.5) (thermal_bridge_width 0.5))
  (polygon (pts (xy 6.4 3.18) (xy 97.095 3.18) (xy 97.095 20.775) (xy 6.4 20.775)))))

